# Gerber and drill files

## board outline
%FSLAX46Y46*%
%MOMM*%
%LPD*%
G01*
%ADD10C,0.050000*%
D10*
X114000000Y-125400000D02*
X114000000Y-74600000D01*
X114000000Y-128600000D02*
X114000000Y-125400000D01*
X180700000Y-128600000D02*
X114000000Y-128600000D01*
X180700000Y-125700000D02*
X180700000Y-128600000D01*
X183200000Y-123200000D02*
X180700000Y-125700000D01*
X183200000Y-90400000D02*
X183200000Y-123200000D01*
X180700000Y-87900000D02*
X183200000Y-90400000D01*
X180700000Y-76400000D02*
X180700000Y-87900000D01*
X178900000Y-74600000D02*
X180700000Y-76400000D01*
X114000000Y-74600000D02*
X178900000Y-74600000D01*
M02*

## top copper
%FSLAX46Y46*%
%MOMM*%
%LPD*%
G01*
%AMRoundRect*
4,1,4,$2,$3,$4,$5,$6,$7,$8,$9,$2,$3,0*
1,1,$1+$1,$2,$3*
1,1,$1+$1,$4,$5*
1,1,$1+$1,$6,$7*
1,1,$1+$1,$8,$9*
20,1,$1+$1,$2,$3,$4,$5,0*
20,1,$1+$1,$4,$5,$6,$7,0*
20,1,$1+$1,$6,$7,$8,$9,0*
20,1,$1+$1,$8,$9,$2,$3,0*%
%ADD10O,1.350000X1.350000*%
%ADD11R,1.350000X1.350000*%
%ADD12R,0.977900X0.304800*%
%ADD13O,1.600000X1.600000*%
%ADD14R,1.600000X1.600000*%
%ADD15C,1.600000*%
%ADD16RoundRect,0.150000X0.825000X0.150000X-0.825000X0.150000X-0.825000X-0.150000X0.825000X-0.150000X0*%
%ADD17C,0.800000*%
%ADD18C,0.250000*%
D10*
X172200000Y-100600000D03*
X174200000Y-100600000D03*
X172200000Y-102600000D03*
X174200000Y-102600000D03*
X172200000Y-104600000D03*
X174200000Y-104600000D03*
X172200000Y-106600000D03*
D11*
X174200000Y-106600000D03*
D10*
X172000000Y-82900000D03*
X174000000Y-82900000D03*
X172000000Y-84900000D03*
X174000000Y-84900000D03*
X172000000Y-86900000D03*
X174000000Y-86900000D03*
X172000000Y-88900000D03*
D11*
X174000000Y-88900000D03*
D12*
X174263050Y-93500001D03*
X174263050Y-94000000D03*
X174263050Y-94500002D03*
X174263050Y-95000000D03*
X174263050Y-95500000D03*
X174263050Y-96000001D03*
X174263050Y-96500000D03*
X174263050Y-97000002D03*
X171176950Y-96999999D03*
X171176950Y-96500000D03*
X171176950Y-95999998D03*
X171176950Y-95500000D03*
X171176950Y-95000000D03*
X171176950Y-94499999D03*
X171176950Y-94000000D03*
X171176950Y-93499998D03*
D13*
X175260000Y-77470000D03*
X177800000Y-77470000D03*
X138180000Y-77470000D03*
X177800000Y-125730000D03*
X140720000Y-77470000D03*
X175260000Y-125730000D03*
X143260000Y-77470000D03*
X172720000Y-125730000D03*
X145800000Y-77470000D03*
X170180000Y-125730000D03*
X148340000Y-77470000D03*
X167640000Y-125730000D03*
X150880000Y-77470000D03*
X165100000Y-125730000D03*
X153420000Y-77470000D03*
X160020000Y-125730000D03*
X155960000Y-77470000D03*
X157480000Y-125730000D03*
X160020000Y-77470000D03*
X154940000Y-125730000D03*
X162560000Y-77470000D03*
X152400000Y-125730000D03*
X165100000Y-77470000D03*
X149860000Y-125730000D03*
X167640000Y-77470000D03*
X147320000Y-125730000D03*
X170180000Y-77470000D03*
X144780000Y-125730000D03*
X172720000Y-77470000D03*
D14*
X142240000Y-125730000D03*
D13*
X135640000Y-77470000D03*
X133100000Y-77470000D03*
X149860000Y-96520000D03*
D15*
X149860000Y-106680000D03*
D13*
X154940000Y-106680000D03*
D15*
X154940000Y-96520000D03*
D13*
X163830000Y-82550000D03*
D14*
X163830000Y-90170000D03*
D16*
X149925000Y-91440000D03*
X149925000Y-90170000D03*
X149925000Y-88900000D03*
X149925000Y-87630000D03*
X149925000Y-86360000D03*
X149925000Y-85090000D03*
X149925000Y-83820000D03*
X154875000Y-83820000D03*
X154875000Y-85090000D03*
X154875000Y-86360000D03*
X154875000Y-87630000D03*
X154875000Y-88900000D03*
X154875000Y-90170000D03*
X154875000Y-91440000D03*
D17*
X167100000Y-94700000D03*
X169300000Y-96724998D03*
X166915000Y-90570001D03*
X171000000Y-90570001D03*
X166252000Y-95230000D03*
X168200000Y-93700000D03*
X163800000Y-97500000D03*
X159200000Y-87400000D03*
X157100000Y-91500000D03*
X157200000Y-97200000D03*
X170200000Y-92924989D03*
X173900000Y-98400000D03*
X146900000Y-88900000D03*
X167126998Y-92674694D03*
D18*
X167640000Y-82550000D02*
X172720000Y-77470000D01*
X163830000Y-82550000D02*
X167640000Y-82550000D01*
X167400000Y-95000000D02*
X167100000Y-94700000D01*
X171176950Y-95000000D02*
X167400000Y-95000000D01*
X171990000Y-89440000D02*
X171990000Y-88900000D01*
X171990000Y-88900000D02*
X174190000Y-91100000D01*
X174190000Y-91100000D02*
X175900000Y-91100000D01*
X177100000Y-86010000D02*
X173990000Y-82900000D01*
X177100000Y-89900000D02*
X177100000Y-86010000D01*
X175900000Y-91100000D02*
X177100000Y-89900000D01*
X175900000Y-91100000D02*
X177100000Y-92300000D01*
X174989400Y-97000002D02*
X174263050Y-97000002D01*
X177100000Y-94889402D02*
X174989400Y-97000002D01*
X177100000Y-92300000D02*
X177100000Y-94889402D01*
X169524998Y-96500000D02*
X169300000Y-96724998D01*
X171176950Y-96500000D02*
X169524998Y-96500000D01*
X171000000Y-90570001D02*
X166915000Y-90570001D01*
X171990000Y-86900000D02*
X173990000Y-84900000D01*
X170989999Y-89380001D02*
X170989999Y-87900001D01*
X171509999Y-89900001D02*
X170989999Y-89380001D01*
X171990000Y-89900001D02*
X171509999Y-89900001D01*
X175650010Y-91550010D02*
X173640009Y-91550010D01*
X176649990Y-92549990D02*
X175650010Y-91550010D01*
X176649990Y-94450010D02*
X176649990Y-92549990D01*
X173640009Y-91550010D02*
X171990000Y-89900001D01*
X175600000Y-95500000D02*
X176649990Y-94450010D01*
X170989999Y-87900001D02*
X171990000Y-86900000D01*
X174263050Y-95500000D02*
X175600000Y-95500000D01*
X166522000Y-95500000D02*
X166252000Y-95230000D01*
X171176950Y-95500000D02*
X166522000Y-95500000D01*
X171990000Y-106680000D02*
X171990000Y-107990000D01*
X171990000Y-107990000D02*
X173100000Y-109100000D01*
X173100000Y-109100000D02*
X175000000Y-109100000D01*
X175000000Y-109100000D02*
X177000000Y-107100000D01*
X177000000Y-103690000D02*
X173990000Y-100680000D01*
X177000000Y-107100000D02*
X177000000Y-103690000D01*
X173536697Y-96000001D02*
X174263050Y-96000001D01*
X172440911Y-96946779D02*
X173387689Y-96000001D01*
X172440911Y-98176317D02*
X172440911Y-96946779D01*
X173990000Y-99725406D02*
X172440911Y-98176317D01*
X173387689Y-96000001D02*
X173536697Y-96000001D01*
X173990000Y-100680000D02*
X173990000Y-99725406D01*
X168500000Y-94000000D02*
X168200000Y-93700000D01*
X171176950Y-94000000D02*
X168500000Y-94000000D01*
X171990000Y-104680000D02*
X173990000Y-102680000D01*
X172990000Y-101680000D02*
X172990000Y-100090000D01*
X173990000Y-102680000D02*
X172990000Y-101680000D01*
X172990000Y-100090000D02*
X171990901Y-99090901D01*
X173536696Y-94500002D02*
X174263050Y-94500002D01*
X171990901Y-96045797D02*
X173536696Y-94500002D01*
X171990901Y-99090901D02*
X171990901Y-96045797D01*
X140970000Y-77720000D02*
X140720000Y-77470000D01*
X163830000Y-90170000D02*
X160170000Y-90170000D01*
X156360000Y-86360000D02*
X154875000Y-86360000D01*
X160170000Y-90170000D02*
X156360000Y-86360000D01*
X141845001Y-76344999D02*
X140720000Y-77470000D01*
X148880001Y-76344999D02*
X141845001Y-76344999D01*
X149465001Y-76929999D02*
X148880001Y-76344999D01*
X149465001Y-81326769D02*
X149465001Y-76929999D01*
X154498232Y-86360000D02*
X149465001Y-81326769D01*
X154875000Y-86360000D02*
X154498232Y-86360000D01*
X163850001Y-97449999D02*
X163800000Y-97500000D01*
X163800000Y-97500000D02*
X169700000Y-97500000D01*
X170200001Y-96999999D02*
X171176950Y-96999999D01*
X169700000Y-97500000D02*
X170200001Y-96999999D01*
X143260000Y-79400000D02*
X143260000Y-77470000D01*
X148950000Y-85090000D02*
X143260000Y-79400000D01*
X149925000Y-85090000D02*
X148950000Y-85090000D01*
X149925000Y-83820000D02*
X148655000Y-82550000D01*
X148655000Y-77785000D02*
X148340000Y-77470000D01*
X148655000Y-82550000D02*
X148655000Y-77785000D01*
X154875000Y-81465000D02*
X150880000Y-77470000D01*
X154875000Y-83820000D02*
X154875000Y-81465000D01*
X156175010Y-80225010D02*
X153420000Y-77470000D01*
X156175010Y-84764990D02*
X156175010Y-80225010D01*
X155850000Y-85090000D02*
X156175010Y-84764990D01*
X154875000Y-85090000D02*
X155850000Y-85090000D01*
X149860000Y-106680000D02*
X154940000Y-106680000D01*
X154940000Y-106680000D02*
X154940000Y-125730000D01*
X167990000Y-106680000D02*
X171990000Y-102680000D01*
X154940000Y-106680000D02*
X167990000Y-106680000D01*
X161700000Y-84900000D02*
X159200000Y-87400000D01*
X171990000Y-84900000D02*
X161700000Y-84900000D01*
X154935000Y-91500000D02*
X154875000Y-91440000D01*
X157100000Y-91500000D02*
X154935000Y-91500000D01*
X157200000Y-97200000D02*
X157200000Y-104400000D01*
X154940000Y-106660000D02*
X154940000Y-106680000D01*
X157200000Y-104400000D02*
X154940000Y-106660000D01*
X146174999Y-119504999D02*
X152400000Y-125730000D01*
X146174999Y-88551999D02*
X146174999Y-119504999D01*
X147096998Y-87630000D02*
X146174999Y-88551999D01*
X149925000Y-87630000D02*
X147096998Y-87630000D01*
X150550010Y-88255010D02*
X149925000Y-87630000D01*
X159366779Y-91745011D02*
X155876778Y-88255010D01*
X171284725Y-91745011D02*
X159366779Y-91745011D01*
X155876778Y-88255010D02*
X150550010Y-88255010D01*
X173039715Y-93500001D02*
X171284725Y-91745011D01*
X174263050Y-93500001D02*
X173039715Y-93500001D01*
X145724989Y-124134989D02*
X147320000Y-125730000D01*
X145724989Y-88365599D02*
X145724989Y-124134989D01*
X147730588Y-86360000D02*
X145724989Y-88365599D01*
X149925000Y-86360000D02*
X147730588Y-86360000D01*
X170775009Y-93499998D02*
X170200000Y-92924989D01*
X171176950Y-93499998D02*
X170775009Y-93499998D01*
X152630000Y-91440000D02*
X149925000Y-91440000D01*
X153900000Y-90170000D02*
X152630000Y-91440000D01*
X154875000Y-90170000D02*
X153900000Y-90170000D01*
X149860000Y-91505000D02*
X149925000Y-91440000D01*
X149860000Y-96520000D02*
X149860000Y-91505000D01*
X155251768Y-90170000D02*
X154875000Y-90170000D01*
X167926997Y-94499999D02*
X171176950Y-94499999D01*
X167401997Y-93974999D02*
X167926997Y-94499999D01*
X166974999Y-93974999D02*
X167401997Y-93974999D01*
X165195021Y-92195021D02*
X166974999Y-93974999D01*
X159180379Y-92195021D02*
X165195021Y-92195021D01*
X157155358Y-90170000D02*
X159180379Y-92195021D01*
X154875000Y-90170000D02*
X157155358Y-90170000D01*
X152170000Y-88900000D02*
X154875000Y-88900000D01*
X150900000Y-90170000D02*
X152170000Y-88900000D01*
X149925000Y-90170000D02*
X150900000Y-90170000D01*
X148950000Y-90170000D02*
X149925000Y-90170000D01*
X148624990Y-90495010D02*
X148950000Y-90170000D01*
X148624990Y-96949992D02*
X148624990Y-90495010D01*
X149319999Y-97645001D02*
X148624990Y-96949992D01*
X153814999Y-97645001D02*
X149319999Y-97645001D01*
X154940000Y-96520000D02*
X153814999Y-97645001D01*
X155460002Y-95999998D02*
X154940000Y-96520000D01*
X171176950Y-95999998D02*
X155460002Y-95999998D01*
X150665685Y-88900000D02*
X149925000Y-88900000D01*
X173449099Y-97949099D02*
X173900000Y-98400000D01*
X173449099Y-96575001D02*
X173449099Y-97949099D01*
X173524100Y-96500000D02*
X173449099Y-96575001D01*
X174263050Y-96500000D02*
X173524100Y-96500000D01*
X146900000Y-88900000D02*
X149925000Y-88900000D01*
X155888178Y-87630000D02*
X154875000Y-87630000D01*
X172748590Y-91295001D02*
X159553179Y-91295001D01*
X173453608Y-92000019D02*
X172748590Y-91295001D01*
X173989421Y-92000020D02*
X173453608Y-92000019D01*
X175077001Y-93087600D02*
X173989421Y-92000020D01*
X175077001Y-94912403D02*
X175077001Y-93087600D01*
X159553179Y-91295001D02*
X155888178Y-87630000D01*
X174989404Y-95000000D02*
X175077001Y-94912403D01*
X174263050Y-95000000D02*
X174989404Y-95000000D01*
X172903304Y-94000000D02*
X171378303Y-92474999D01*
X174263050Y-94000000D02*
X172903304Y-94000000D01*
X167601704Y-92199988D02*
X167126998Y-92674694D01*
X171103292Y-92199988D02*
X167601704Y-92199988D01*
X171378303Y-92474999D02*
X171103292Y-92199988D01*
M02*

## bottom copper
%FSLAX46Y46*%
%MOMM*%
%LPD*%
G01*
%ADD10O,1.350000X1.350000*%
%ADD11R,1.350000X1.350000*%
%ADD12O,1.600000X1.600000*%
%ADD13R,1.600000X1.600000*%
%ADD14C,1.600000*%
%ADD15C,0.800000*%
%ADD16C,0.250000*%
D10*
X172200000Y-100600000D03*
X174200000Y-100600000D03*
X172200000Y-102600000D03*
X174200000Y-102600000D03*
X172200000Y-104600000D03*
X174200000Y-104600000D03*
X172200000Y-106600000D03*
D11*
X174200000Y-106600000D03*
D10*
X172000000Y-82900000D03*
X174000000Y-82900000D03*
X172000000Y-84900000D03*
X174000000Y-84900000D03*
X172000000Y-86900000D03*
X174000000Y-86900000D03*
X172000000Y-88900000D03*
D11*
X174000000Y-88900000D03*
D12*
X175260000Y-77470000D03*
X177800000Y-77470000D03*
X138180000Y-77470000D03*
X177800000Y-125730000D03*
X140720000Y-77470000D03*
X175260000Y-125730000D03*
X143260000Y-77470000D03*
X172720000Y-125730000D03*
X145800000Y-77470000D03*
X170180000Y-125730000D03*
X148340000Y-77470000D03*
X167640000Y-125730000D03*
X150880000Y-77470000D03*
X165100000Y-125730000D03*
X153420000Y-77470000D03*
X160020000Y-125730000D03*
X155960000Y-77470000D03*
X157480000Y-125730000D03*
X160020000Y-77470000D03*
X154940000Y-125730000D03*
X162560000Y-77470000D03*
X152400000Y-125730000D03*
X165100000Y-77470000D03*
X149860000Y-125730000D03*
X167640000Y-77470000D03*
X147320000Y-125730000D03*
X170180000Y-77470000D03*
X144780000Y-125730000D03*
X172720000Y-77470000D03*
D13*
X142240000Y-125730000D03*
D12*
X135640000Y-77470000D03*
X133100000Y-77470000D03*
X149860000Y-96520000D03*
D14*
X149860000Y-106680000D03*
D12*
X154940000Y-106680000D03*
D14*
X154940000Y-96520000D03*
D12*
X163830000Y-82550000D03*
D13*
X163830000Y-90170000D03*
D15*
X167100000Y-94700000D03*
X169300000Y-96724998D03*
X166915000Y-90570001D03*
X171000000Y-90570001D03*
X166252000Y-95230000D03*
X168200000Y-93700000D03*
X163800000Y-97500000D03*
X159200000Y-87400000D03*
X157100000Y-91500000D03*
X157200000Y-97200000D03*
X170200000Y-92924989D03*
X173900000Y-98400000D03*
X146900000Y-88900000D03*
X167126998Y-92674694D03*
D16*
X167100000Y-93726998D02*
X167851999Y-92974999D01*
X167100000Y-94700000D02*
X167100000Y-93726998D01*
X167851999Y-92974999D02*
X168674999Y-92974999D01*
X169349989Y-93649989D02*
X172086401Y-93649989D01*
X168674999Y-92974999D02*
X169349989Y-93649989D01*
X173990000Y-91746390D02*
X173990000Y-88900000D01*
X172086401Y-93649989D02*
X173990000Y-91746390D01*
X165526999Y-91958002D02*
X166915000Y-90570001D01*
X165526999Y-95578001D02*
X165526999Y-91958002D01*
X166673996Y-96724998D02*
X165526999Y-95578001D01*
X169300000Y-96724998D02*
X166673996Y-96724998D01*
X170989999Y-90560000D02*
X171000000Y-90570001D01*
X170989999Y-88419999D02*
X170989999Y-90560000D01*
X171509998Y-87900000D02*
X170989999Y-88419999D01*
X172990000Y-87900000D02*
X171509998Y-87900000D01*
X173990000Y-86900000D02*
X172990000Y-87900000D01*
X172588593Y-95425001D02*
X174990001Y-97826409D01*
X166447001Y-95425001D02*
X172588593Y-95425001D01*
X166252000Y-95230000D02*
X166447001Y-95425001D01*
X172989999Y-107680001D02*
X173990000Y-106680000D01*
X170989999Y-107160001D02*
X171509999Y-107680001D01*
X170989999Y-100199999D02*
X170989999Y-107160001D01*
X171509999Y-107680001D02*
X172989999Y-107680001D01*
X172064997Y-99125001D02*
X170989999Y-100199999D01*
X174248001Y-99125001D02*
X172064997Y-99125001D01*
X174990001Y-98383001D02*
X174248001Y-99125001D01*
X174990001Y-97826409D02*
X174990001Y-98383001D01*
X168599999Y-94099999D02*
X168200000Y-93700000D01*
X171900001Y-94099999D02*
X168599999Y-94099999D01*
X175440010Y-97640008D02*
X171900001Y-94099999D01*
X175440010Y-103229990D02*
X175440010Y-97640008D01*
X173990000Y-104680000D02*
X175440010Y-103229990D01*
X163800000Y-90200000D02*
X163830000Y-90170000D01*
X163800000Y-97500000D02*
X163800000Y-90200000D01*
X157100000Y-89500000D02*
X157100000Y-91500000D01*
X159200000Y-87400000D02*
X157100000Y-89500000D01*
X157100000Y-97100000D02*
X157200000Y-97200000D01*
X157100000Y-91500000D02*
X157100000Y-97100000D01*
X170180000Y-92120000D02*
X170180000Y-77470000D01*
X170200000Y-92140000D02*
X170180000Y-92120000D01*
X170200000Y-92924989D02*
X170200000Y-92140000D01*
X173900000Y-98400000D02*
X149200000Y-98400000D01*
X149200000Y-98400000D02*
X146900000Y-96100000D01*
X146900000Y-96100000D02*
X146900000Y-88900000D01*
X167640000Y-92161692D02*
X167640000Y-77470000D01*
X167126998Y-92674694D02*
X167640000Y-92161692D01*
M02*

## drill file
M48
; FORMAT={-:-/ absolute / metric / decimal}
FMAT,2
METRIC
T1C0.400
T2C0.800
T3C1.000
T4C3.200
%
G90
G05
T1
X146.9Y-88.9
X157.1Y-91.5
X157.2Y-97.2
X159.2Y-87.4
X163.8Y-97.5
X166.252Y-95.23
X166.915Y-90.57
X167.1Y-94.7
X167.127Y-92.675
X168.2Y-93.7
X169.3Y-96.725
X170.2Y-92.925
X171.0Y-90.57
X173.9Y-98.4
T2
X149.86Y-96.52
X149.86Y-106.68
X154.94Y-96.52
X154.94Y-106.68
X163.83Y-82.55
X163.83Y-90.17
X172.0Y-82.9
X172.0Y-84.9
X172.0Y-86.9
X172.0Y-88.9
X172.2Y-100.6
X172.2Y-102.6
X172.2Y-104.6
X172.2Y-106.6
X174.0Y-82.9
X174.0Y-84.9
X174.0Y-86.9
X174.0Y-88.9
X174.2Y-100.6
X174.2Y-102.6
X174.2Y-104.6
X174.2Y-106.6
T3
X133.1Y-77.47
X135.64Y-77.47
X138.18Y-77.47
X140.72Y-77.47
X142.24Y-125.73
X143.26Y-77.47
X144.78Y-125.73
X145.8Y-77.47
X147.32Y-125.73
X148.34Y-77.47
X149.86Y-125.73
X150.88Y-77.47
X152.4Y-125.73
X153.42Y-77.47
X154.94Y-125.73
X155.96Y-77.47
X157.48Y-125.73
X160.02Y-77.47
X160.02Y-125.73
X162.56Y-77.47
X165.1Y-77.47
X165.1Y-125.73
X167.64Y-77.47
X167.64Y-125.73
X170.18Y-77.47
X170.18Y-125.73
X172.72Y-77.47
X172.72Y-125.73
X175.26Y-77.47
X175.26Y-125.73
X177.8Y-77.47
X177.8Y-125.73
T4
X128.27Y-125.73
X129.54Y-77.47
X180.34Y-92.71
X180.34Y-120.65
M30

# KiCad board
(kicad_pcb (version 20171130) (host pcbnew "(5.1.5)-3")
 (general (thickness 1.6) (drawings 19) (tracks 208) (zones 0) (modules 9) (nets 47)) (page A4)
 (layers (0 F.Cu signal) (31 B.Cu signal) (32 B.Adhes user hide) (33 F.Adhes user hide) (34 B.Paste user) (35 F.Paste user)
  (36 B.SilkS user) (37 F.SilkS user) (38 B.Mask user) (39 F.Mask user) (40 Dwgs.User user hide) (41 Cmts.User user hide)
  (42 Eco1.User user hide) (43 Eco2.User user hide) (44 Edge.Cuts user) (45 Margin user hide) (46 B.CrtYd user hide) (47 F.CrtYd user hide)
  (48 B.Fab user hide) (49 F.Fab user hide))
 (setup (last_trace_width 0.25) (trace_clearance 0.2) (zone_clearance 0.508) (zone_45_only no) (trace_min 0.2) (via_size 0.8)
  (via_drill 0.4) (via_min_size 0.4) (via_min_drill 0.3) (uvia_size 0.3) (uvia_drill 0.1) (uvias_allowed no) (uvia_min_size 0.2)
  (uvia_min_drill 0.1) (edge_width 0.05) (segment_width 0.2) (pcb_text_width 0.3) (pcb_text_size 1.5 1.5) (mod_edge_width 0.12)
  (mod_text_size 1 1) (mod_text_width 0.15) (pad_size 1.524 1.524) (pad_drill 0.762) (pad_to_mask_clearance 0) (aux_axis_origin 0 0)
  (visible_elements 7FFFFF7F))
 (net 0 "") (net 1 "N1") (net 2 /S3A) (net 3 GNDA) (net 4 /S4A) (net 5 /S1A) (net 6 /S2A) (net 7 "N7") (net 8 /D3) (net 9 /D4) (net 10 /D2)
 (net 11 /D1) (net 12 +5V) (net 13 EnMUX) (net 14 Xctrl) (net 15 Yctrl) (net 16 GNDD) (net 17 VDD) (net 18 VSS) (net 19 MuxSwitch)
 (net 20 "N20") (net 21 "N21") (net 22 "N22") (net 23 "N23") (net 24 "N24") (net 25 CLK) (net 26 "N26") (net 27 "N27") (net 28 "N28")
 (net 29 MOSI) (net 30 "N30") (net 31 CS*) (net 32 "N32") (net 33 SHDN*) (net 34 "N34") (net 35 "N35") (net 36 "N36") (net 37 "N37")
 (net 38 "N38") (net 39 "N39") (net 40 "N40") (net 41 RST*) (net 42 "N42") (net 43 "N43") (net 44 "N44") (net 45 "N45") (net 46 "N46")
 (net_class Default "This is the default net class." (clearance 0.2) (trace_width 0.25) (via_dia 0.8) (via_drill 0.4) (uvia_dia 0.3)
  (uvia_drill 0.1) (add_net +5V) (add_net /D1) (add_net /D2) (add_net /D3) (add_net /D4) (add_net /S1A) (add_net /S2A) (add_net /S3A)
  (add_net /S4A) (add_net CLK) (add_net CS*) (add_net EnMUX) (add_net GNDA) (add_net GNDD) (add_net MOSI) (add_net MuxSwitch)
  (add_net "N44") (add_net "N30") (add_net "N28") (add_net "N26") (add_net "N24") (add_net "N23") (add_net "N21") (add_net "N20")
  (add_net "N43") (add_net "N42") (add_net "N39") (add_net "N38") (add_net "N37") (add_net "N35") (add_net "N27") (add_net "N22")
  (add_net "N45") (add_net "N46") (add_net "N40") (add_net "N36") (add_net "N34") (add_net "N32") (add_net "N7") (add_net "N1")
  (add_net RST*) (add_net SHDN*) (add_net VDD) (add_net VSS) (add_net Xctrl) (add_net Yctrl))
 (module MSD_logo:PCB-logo (layer F.Cu) (at 128.7 102 90)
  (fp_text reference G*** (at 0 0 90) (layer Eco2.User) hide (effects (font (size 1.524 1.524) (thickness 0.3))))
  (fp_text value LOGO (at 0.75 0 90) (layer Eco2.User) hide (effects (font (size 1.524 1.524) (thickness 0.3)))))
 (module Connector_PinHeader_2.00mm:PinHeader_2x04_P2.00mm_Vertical (layer F.Cu) (at 174.2 106.6 180)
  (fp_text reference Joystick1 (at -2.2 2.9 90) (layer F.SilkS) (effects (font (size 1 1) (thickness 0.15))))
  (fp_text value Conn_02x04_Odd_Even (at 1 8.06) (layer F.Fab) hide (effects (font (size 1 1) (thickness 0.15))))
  (pad 8 thru_hole oval (at 2 6 180) (size 1.35 1.35) (drill 0.8) (layers *.Cu *.Mask) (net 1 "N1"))
  (pad 7 thru_hole oval (at 0 6 180) (size 1.35 1.35) (drill 0.8) (layers *.Cu *.Mask) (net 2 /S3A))
  (pad 6 thru_hole oval (at 2 4 180) (size 1.35 1.35) (drill 0.8) (layers *.Cu *.Mask) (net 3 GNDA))
  (pad 5 thru_hole oval (at 0 4 180) (size 1.35 1.35) (drill 0.8) (layers *.Cu *.Mask) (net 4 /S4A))
  (pad 4 thru_hole oval (at 2 2 180) (size 1.35 1.35) (drill 0.8) (layers *.Cu *.Mask) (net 4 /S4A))
  (pad 3 thru_hole oval (at 0 2 180) (size 1.35 1.35) (drill 0.8) (layers *.Cu *.Mask) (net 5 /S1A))
  (pad 2 thru_hole oval (at 2 0 180) (size 1.35 1.35) (drill 0.8) (layers *.Cu *.Mask) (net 2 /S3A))
  (pad 1 thru_hole rect (at 0 0 180) (size 1.35 1.35) (drill 0.8) (layers *.Cu *.Mask) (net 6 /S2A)))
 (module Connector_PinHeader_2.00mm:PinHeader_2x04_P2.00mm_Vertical (layer F.Cu) (at 174 88.9 180)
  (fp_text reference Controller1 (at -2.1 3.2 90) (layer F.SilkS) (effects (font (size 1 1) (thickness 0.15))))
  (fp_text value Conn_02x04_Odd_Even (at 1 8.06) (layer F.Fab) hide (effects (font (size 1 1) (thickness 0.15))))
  (pad 8 thru_hole oval (at 2 6 180) (size 1.35 1.35) (drill 0.8) (layers *.Cu *.Mask) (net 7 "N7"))
  (pad 7 thru_hole oval (at 0 6 180) (size 1.35 1.35) (drill 0.8) (layers *.Cu *.Mask) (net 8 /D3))
  (pad 6 thru_hole oval (at 2 4 180) (size 1.35 1.35) (drill 0.8) (layers *.Cu *.Mask) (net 3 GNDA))
  (pad 5 thru_hole oval (at 0 4 180) (size 1.35 1.35) (drill 0.8) (layers *.Cu *.Mask) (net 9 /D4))
  (pad 4 thru_hole oval (at 2 2 180) (size 1.35 1.35) (drill 0.8) (layers *.Cu *.Mask) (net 9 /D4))
  (pad 3 thru_hole oval (at 0 2 180) (size 1.35 1.35) (drill 0.8) (layers *.Cu *.Mask) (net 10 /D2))
  (pad 2 thru_hole oval (at 2 0 180) (size 1.35 1.35) (drill 0.8) (layers *.Cu *.Mask) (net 8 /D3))
  (pad 1 thru_hole rect (at 0 0 180) (size 1.35 1.35) (drill 0.8) (layers *.Cu *.Mask) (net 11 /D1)))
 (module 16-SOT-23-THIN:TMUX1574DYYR (layer F.Cu) (at 172.72 95.25)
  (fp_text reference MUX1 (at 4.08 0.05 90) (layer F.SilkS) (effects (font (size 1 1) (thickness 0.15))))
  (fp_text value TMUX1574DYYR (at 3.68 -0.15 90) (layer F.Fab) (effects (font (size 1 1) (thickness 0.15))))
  (pad 16 smd rect (at 1.54305 -1.749999) (size 0.9779 0.3048) (layers F.Cu F.Paste F.Mask) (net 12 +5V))
  (pad 15 smd rect (at 1.54305 -1.25) (size 0.9779 0.3048) (layers F.Cu F.Paste F.Mask) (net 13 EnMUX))
  (pad 14 smd rect (at 1.54305 -0.749998) (size 0.9779 0.3048) (layers F.Cu F.Paste F.Mask) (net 4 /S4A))
  (pad 13 smd rect (at 1.54305 -0.25) (size 0.9779 0.3048) (layers F.Cu F.Paste F.Mask) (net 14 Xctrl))
  (pad 12 smd rect (at 1.54305 0.25) (size 0.9779 0.3048) (layers F.Cu F.Paste F.Mask) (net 9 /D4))
  (pad 11 smd rect (at 1.54305 0.750001) (size 0.9779 0.3048) (layers F.Cu F.Paste F.Mask) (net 2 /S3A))
  (pad 10 smd rect (at 1.54305 1.25) (size 0.9779 0.3048) (layers F.Cu F.Paste F.Mask) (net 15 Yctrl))
  (pad 9 smd rect (at 1.54305 1.750002) (size 0.9779 0.3048) (layers F.Cu F.Paste F.Mask) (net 8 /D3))
  (pad 8 smd rect (at -1.54305 1.749999) (size 0.9779 0.3048) (layers F.Cu F.Paste F.Mask) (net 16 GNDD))
  (pad 7 smd rect (at -1.54305 1.25) (size 0.9779 0.3048) (layers F.Cu F.Paste F.Mask) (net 10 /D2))
  (pad 6 smd rect (at -1.54305 0.749998) (size 0.9779 0.3048) (layers F.Cu F.Paste F.Mask) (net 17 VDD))
  (pad 5 smd rect (at -1.54305 0.25) (size 0.9779 0.3048) (layers F.Cu F.Paste F.Mask) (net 6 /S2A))
  (pad 4 smd rect (at -1.54305 -0.25) (size 0.9779 0.3048) (layers F.Cu F.Paste F.Mask) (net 11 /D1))
  (pad 3 smd rect (at -1.54305 -0.750001) (size 0.9779 0.3048) (layers F.Cu F.Paste F.Mask) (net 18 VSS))
  (pad 2 smd rect (at -1.54305 -1.25) (size 0.9779 0.3048) (layers F.Cu F.Paste F.Mask) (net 5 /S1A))
  (pad 1 smd rect (at -1.54305 -1.750002) (size 0.9779 0.3048) (layers F.Cu F.Paste F.Mask) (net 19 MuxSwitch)))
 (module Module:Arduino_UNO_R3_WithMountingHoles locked (layer B.Cu) (at 142.24 125.73)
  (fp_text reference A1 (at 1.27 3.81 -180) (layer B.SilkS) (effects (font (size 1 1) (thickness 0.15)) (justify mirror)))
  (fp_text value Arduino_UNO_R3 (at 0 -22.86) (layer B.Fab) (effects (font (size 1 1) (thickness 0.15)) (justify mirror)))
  (pad "" np_thru_hole circle (at 38.1 -5.08 270) (size 3.2 3.2) (drill 3.2) (layers *.Cu *.Mask))
  (pad "" np_thru_hole circle (at 38.1 -33.02 270) (size 3.2 3.2) (drill 3.2) (layers *.Cu *.Mask))
  (pad "" np_thru_hole circle (at -12.7 -48.26 270) (size 3.2 3.2) (drill 3.2) (layers *.Cu *.Mask))
  (pad "" np_thru_hole circle (at -13.97 0 270) (size 3.2 3.2) (drill 3.2) (layers *.Cu *.Mask))
  (pad 16 thru_hole oval (at 33.02 -48.26 270) (size 1.6 1.6) (drill 1) (layers *.Cu *.Mask) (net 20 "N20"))
  (pad 15 thru_hole oval (at 35.56 -48.26 270) (size 1.6 1.6) (drill 1) (layers *.Cu *.Mask) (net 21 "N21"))
  (pad 30 thru_hole oval (at -4.06 -48.26 270) (size 1.6 1.6) (drill 1) (layers *.Cu *.Mask) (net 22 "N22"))
  (pad 14 thru_hole oval (at 35.56 0 270) (size 1.6 1.6) (drill 1) (layers *.Cu *.Mask) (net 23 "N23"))
  (pad 29 thru_hole oval (at -1.52 -48.26 270) (size 1.6 1.6) (drill 1) (layers *.Cu *.Mask) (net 16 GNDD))
  (pad 13 thru_hole oval (at 33.02 0 270) (size 1.6 1.6) (drill 1) (layers *.Cu *.Mask) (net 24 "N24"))
  (pad 28 thru_hole oval (at 1.02 -48.26 270) (size 1.6 1.6) (drill 1) (layers *.Cu *.Mask) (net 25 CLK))
  (pad 12 thru_hole oval (at 30.48 0 270) (size 1.6 1.6) (drill 1) (layers *.Cu *.Mask) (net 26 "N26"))
  (pad 27 thru_hole oval (at 3.56 -48.26 270) (size 1.6 1.6) (drill 1) (layers *.Cu *.Mask) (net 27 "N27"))
  (pad 11 thru_hole oval (at 27.94 0 270) (size 1.6 1.6) (drill 1) (layers *.Cu *.Mask) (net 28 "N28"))
  (pad 26 thru_hole oval (at 6.1 -48.26 270) (size 1.6 1.6) (drill 1) (layers *.Cu *.Mask) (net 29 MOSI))
  (pad 10 thru_hole oval (at 25.4 0 270) (size 1.6 1.6) (drill 1) (layers *.Cu *.Mask) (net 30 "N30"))
  (pad 25 thru_hole oval (at 8.64 -48.26 270) (size 1.6 1.6) (drill 1) (layers *.Cu *.Mask) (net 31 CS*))
  (pad 9 thru_hole oval (at 22.86 0 270) (size 1.6 1.6) (drill 1) (layers *.Cu *.Mask) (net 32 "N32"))
  (pad 24 thru_hole oval (at 11.18 -48.26 270) (size 1.6 1.6) (drill 1) (layers *.Cu *.Mask) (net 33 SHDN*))
  (pad 8 thru_hole oval (at 17.78 0 270) (size 1.6 1.6) (drill 1) (layers *.Cu *.Mask) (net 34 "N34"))
  (pad 23 thru_hole oval (at 13.72 -48.26 270) (size 1.6 1.6) (drill 1) (layers *.Cu *.Mask) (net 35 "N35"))
  (pad 7 thru_hole oval (at 15.24 0 270) (size 1.6 1.6) (drill 1) (layers *.Cu *.Mask) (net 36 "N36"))
  (pad 22 thru_hole oval (at 17.78 -48.26 270) (size 1.6 1.6) (drill 1) (layers *.Cu *.Mask) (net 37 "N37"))
  (pad 6 thru_hole oval (at 12.7 0 270) (size 1.6 1.6) (drill 1) (layers *.Cu *.Mask) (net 3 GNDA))
  (pad 21 thru_hole oval (at 20.32 -48.26 270) (size 1.6 1.6) (drill 1) (layers *.Cu *.Mask) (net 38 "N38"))
  (pad 5 thru_hole oval (at 10.16 0 270) (size 1.6 1.6) (drill 1) (layers *.Cu *.Mask) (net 12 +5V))
  (pad 20 thru_hole oval (at 22.86 -48.26 270) (size 1.6 1.6) (drill 1) (layers *.Cu *.Mask) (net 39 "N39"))
  (pad 4 thru_hole oval (at 7.62 0 270) (size 1.6 1.6) (drill 1) (layers *.Cu *.Mask) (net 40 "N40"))
  (pad 19 thru_hole oval (at 25.4 -48.26 270) (size 1.6 1.6) (drill 1) (layers *.Cu *.Mask) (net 13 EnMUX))
  (pad 3 thru_hole oval (at 5.08 0 270) (size 1.6 1.6) (drill 1) (layers *.Cu *.Mask) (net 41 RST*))
  (pad 18 thru_hole oval (at 27.94 -48.26 270) (size 1.6 1.6) (drill 1) (layers *.Cu *.Mask) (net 19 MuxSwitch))
  (pad 2 thru_hole oval (at 2.54 0 270) (size 1.6 1.6) (drill 1) (layers *.Cu *.Mask) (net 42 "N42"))
  (pad 17 thru_hole oval (at 30.48 -48.26 270) (size 1.6 1.6) (drill 1) (layers *.Cu *.Mask) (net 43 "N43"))
  (pad 1 thru_hole rect (at 0 0 270) (size 1.6 1.6) (drill 1) (layers *.Cu *.Mask) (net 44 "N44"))
  (pad 31 thru_hole oval (at -6.6 -48.26 270) (size 1.6 1.6) (drill 1) (layers *.Cu *.Mask) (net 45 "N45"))
  (pad 32 thru_hole oval (at -9.14 -48.26 270) (size 1.6 1.6) (drill 1) (layers *.Cu *.Mask) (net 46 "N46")))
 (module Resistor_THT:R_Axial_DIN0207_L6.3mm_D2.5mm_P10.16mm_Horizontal (layer F.Cu) (at 149.86 106.68 90)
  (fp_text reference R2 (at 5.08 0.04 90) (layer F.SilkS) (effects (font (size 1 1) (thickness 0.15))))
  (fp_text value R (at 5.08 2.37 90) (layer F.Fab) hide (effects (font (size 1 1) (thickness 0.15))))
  (pad 2 thru_hole oval (at 10.16 0 90) (size 1.6 1.6) (drill 0.8) (layers *.Cu *.Mask) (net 18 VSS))
  (pad 1 thru_hole circle (at 0 0 90) (size 1.6 1.6) (drill 0.8) (layers *.Cu *.Mask) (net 3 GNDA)))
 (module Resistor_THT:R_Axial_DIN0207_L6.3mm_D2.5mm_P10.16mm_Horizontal (layer F.Cu) (at 154.94 96.52 270)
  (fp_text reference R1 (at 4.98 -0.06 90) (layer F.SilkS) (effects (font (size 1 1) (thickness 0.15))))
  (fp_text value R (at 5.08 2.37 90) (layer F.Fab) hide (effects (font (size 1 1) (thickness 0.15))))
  (pad 2 thru_hole oval (at 10.16 0 270) (size 1.6 1.6) (drill 0.8) (layers *.Cu *.Mask) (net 3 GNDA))
  (pad 1 thru_hole circle (at 0 0 270) (size 1.6 1.6) (drill 0.8) (layers *.Cu *.Mask) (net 17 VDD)))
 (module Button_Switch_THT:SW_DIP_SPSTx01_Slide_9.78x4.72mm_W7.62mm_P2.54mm (layer F.Cu) (at 163.83 90.17 90)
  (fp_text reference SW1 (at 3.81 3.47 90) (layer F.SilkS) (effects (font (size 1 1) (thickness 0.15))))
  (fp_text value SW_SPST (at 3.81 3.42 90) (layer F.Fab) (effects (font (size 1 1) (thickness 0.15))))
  (pad 2 thru_hole oval (at 7.62 0 90) (size 1.6 1.6) (drill 0.8) (layers *.Cu *.Mask) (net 43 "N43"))
  (pad 1 thru_hole rect (at 0 0 90) (size 1.6 1.6) (drill 0.8) (layers *.Cu *.Mask) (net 16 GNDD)))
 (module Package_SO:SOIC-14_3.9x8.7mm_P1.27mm (layer F.Cu) (at 152.4 87.63 180)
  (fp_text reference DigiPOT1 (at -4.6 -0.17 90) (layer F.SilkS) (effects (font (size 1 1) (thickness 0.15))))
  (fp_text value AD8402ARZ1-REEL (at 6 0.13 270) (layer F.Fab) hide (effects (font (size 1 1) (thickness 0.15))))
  (pad 14 smd roundrect (at 2.475 -3.81 180) (size 1.95 0.6) (layers F.Cu F.Paste F.Mask) (roundrect_rratio 0.25) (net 18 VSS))
  (pad 13 smd roundrect (at 2.475 -2.54 180) (size 1.95 0.6) (layers F.Cu F.Paste F.Mask) (roundrect_rratio 0.25) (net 17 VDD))
  (pad 12 smd roundrect (at 2.475 -1.27 180) (size 1.95 0.6) (layers F.Cu F.Paste F.Mask) (roundrect_rratio 0.25) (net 15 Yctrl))
  (pad 11 smd roundrect (at 2.475 0 180) (size 1.95 0.6) (layers F.Cu F.Paste F.Mask) (roundrect_rratio 0.25) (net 12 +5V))
  (pad 10 smd roundrect (at 2.475 1.27 180) (size 1.95 0.6) (layers F.Cu F.Paste F.Mask) (roundrect_rratio 0.25) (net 41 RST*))
  (pad 9 smd roundrect (at 2.475 2.54 180) (size 1.95 0.6) (layers F.Cu F.Paste F.Mask) (roundrect_rratio 0.25) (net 25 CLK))
  (pad 8 smd roundrect (at 2.475 3.81 180) (size 1.95 0.6) (layers F.Cu F.Paste F.Mask) (roundrect_rratio 0.25) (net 29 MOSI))
  (pad 7 smd roundrect (at -2.475 3.81 180) (size 1.95 0.6) (layers F.Cu F.Paste F.Mask) (roundrect_rratio 0.25) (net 31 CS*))
  (pad 6 smd roundrect (at -2.475 2.54 180) (size 1.95 0.6) (layers F.Cu F.Paste F.Mask) (roundrect_rratio 0.25) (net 33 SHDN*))
  (pad 5 smd roundrect (at -2.475 1.27 180) (size 1.95 0.6) (layers F.Cu F.Paste F.Mask) (roundrect_rratio 0.25) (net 16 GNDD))
  (pad 4 smd roundrect (at -2.475 0 180) (size 1.95 0.6) (layers F.Cu F.Paste F.Mask) (roundrect_rratio 0.25) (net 14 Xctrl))
  (pad 3 smd roundrect (at -2.475 -1.27 180) (size 1.95 0.6) (layers F.Cu F.Paste F.Mask) (roundrect_rratio 0.25) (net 17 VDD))
  (pad 2 smd roundrect (at -2.475 -2.54 180) (size 1.95 0.6) (layers F.Cu F.Paste F.Mask) (roundrect_rratio 0.25) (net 18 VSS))
  (pad 1 smd roundrect (at -2.475 -3.81 180) (size 1.95 0.6) (layers F.Cu F.Paste F.Mask) (roundrect_rratio 0.25) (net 3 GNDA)))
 (gr_line (start 114 125.4) (end 114 74.6) (layer Edge.Cuts) (width 0.05))
 (gr_line (start 114 128.6) (end 114 125.4) (layer Edge.Cuts) (width 0.05))
 (gr_line (start 180.7 128.6) (end 114 128.6) (layer Edge.Cuts) (width 0.05))
 (gr_line (start 180.7 125.7) (end 180.7 128.6) (layer Edge.Cuts) (width 0.05))
 (gr_line (start 183.2 123.2) (end 180.7 125.7) (layer Edge.Cuts) (width 0.05))
 (gr_line (start 183.2 90.4) (end 183.2 123.2) (layer Edge.Cuts) (width 0.05))
 (gr_line (start 180.7 87.9) (end 183.2 90.4) (layer Edge.Cuts) (width 0.05))
 (gr_line (start 180.7 76.4) (end 180.7 87.9) (layer Edge.Cuts) (width 0.05))
 (gr_line (start 178.9 74.6) (end 180.7 76.4) (layer Edge.Cuts) (width 0.05))
 (gr_line (start 114 74.6) (end 178.9 74.6) (layer Edge.Cuts) (width 0.05))
 (segment (start 167.64 82.55) (end 172.72 77.47) (width 0.25) (layer F.Cu) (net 43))
 (segment (start 163.83 82.55) (end 167.64 82.55) (width 0.25) (layer F.Cu) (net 43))
 (via (at 167.1 94.7) (size 0.8) (drill 0.4) (layers F.Cu B.Cu) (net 11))
 (segment (start 167.4 95) (end 167.1 94.7) (width 0.25) (layer F.Cu) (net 11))
 (segment (start 171.17695 95) (end 167.4 95) (width 0.25) (layer F.Cu) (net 11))
 (segment (start 167.1 93.726998) (end 167.851999 92.974999) (width 0.25) (layer B.Cu) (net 11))
 (segment (start 167.1 94.7) (end 167.1 93.726998) (width 0.25) (layer B.Cu) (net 11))
 (segment (start 167.851999 92.974999) (end 168.674999 92.974999) (width 0.25) (layer B.Cu) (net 11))
 (segment (start 169.349989 93.649989) (end 172.086401 93.649989) (width 0.25) (layer B.Cu) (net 11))
 (segment (start 168.674999 92.974999) (end 169.349989 93.649989) (width 0.25) (layer B.Cu) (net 11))
 (segment (start 173.99 91.74639) (end 173.99 88.9) (width 0.25) (layer B.Cu) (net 11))
 (segment (start 172.086401 93.649989) (end 173.99 91.74639) (width 0.25) (layer B.Cu) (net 11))
 (segment (start 171.99 89.44) (end 171.99 88.9) (width 0.25) (layer F.Cu) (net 8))
 (segment (start 171.99 88.9) (end 174.19 91.1) (width 0.25) (layer F.Cu) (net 8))
 (segment (start 174.19 91.1) (end 175.9 91.1) (width 0.25) (layer F.Cu) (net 8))
 (segment (start 177.1 86.01) (end 173.99 82.9) (width 0.25) (layer F.Cu) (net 8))
 (segment (start 177.1 89.9) (end 177.1 86.01) (width 0.25) (layer F.Cu) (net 8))
 (segment (start 175.9 91.1) (end 177.1 89.9) (width 0.25) (layer F.Cu) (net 8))
 (segment (start 175.9 91.1) (end 177.1 92.3) (width 0.25) (layer F.Cu) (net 8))
 (segment (start 174.9894 97.000002) (end 174.26305 97.000002) (width 0.25) (layer F.Cu) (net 8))
 (segment (start 177.1 94.889402) (end 174.9894 97.000002) (width 0.25) (layer F.Cu) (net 8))
 (segment (start 177.1 92.3) (end 177.1 94.889402) (width 0.25) (layer F.Cu) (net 8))
 (via (at 169.3 96.724998) (size 0.8) (drill 0.4) (layers F.Cu B.Cu) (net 10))
 (segment (start 169.524998 96.5) (end 169.3 96.724998) (width 0.25) (layer F.Cu) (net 10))
 (segment (start 171.17695 96.5) (end 169.524998 96.5) (width 0.25) (layer F.Cu) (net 10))
 (segment (start 165.526999 91.958002) (end 166.915 90.570001) (width 0.25) (layer B.Cu) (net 10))
 (via (at 166.915 90.570001) (size 0.8) (drill 0.4) (layers F.Cu B.Cu) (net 10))
 (segment (start 165.526999 95.578001) (end 165.526999 91.958002) (width 0.25) (layer B.Cu) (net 10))
 (segment (start 166.673996 96.724998) (end 165.526999 95.578001) (width 0.25) (layer B.Cu) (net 10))
 (segment (start 169.3 96.724998) (end 166.673996 96.724998) (width 0.25) (layer B.Cu) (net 10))
 (via (at 171 90.570001) (size 0.8) (drill 0.4) (layers F.Cu B.Cu) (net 10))
 (segment (start 170.989999 90.56) (end 171 90.570001) (width 0.25) (layer B.Cu) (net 10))
 (segment (start 170.989999 88.419999) (end 170.989999 90.56) (width 0.25) (layer B.Cu) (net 10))
 (segment (start 171.509998 87.9) (end 170.989999 88.419999) (width 0.25) (layer B.Cu) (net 10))
 (segment (start 172.99 87.9) (end 171.509998 87.9) (width 0.25) (layer B.Cu) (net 10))
 (segment (start 173.99 86.9) (end 172.99 87.9) (width 0.25) (layer B.Cu) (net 10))
 (segment (start 171 90.570001) (end 166.915 90.570001) (width 0.25) (layer F.Cu) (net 10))
 (segment (start 171.99 86.9) (end 173.99 84.9) (width 0.25) (layer F.Cu) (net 9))
 (segment (start 170.989999 89.380001) (end 170.989999 87.900001) (width 0.25) (layer F.Cu) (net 9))
 (segment (start 171.509999 89.900001) (end 170.989999 89.380001) (width 0.25) (layer F.Cu) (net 9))
 (segment (start 171.99 89.900001) (end 171.509999 89.900001) (width 0.25) (layer F.Cu) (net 9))
 (segment (start 175.65001 91.55001) (end 173.640009 91.55001) (width 0.25) (layer F.Cu) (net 9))
 (segment (start 176.64999 92.54999) (end 175.65001 91.55001) (width 0.25) (layer F.Cu) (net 9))
 (segment (start 176.64999 94.45001) (end 176.64999 92.54999) (width 0.25) (layer F.Cu) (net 9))
 (segment (start 173.640009 91.55001) (end 171.99 89.900001) (width 0.25) (layer F.Cu) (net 9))
 (segment (start 175.6 95.5) (end 176.64999 94.45001) (width 0.25) (layer F.Cu) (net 9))
 (segment (start 170.989999 87.900001) (end 171.99 86.9) (width 0.25) (layer F.Cu) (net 9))
 (segment (start 174.26305 95.5) (end 175.6 95.5) (width 0.25) (layer F.Cu) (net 9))
 (via (at 166.252 95.23) (size 0.8) (drill 0.4) (layers F.Cu B.Cu) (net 6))
 (segment (start 166.522 95.5) (end 166.252 95.23) (width 0.25) (layer F.Cu) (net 6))
 (segment (start 171.17695 95.5) (end 166.522 95.5) (width 0.25) (layer F.Cu) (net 6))
 (segment (start 172.588593 95.425001) (end 174.990001 97.826409) (width 0.25) (layer B.Cu) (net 6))
 (segment (start 166.447001 95.425001) (end 172.588593 95.425001) (width 0.25) (layer B.Cu) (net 6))
 (segment (start 166.252 95.23) (end 166.447001 95.425001) (width 0.25) (layer B.Cu) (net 6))
 (segment (start 172.989999 107.680001) (end 173.99 106.68) (width 0.25) (layer B.Cu) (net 6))
 (segment (start 170.989999 107.160001) (end 171.509999 107.680001) (width 0.25) (layer B.Cu) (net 6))
 (segment (start 170.989999 100.199999) (end 170.989999 107.160001) (width 0.25) (layer B.Cu) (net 6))
 (segment (start 171.509999 107.680001) (end 172.989999 107.680001) (width 0.25) (layer B.Cu) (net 6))
 (segment (start 172.064997 99.125001) (end 170.989999 100.199999) (width 0.25) (layer B.Cu) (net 6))
 (segment (start 174.248001 99.125001) (end 172.064997 99.125001) (width 0.25) (layer B.Cu) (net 6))
 (segment (start 174.990001 98.383001) (end 174.248001 99.125001) (width 0.25) (layer B.Cu) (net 6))
 (segment (start 174.990001 97.826409) (end 174.990001 98.383001) (width 0.25) (layer B.Cu) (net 6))
 (segment (start 171.99 106.68) (end 171.99 107.99) (width 0.25) (layer F.Cu) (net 2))
 (segment (start 171.99 107.99) (end 173.1 109.1) (width 0.25) (layer F.Cu) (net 2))
 (segment (start 173.1 109.1) (end 175 109.1) (width 0.25) (layer F.Cu) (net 2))
 (segment (start 175 109.1) (end 177 107.1) (width 0.25) (layer F.Cu) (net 2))
 (segment (start 177 103.69) (end 173.99 100.68) (width 0.25) (layer F.Cu) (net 2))
 (segment (start 177 107.1) (end 177 103.69) (width 0.25) (layer F.Cu) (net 2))
 (segment (start 173.536697 96.000001) (end 174.26305 96.000001) (width 0.25) (layer F.Cu) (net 2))
 (segment (start 172.440911 96.946779) (end 173.387689 96.000001) (width 0.25) (layer F.Cu) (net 2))
 (segment (start 172.440911 98.176317) (end 172.440911 96.946779) (width 0.25) (layer F.Cu) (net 2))
 (segment (start 173.99 99.725406) (end 172.440911 98.176317) (width 0.25) (layer F.Cu) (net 2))
 (segment (start 173.387689 96.000001) (end 173.536697 96.000001) (width 0.25) (layer F.Cu) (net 2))
 (segment (start 173.99 100.68) (end 173.99 99.725406) (width 0.25) (layer F.Cu) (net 2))
 (via (at 168.2 93.7) (size 0.8) (drill 0.4) (layers F.Cu B.Cu) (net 5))
 (segment (start 168.5 94) (end 168.2 93.7) (width 0.25) (layer F.Cu) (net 5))
 (segment (start 171.17695 94) (end 168.5 94) (width 0.25) (layer F.Cu) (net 5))
 (segment (start 168.599999 94.099999) (end 168.2 93.7) (width 0.25) (layer B.Cu) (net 5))
 (segment (start 171.900001 94.099999) (end 168.599999 94.099999) (width 0.25) (layer B.Cu) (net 5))
 (segment (start 175.44001 97.640008) (end 171.900001 94.099999) (width 0.25) (layer B.Cu) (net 5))
 (segment (start 175.44001 103.22999) (end 175.44001 97.640008) (width 0.25) (layer B.Cu) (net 5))
 (segment (start 173.99 104.68) (end 175.44001 103.22999) (width 0.25) (layer B.Cu) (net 5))
 (segment (start 171.99 104.68) (end 173.99 102.68) (width 0.25) (layer F.Cu) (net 4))
 (segment (start 172.99 101.68) (end 172.99 100.09) (width 0.25) (layer F.Cu) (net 4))
 (segment (start 173.99 102.68) (end 172.99 101.68) (width 0.25) (layer F.Cu) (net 4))
 (segment (start 172.99 100.09) (end 171.990901 99.090901) (width 0.25) (layer F.Cu) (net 4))
 (segment (start 173.536696 94.500002) (end 174.26305 94.500002) (width 0.25) (layer F.Cu) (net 4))
 (segment (start 171.990901 96.045797) (end 173.536696 94.500002) (width 0.25) (layer F.Cu) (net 4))
 (segment (start 171.990901 99.090901) (end 171.990901 96.045797) (width 0.25) (layer F.Cu) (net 4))
 (segment (start 140.97 77.72) (end 140.72 77.47) (width 0.25) (layer F.Cu) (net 16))
 (segment (start 163.83 90.17) (end 160.17 90.17) (width 0.25) (layer F.Cu) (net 16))
 (segment (start 156.36 86.36) (end 154.875 86.36) (width 0.25) (layer F.Cu) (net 16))
 (segment (start 160.17 90.17) (end 156.36 86.36) (width 0.25) (layer F.Cu) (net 16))
 (segment (start 141.845001 76.344999) (end 140.72 77.47) (width 0.25) (layer F.Cu) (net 16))
 (segment (start 148.880001 76.344999) (end 141.845001 76.344999) (width 0.25) (layer F.Cu) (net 16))
 (segment (start 149.465001 76.929999) (end 148.880001 76.344999) (width 0.25) (layer F.Cu) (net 16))
 (segment (start 149.465001 81.326769) (end 149.465001 76.929999) (width 0.25) (layer F.Cu) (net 16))
 (segment (start 154.498232 86.36) (end 149.465001 81.326769) (width 0.25) (layer F.Cu) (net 16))
 (segment (start 154.875 86.36) (end 154.498232 86.36) (width 0.25) (layer F.Cu) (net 16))
 (via (at 163.8 97.5) (size 0.8) (drill 0.4) (layers F.Cu B.Cu) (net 16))
 (segment (start 163.850001 97.449999) (end 163.8 97.5) (width 0.25) (layer F.Cu) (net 16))
 (segment (start 163.8 90.2) (end 163.83 90.17) (width 0.25) (layer B.Cu) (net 16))
 (segment (start 163.8 97.5) (end 163.8 90.2) (width 0.25) (layer B.Cu) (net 16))
 (segment (start 163.8 97.5) (end 169.7 97.5) (width 0.25) (layer F.Cu) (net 16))
 (segment (start 170.200001 96.999999) (end 171.17695 96.999999) (width 0.25) (layer F.Cu) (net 16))
 (segment (start 169.7 97.5) (end 170.200001 96.999999) (width 0.25) (layer F.Cu) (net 16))
 (segment (start 143.26 79.4) (end 143.26 77.47) (width 0.25) (layer F.Cu) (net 25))
 (segment (start 148.95 85.09) (end 143.26 79.4) (width 0.25) (layer F.Cu) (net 25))
 (segment (start 149.925 85.09) (end 148.95 85.09) (width 0.25) (layer F.Cu) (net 25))
 (segment (start 149.925 83.82) (end 148.655 82.55) (width 0.25) (layer F.Cu) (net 29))
 (segment (start 148.655 77.785) (end 148.34 77.47) (width 0.25) (layer F.Cu) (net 29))
 (segment (start 148.655 82.55) (end 148.655 77.785) (width 0.25) (layer F.Cu) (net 29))
 (segment (start 154.875 81.465) (end 150.88 77.47) (width 0.25) (layer F.Cu) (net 31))
 (segment (start 154.875 83.82) (end 154.875 81.465) (width 0.25) (layer F.Cu) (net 31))
 (segment (start 156.17501 80.22501) (end 153.42 77.47) (width 0.25) (layer F.Cu) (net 33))
 (segment (start 156.17501 84.76499) (end 156.17501 80.22501) (width 0.25) (layer F.Cu) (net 33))
 (segment (start 155.85 85.09) (end 156.17501 84.76499) (width 0.25) (layer F.Cu) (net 33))
 (segment (start 154.875 85.09) (end 155.85 85.09) (width 0.25) (layer F.Cu) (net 33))
 (segment (start 149.86 106.68) (end 154.94 106.68) (width 0.25) (layer F.Cu) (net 3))
 (segment (start 154.94 106.68) (end 154.94 125.73) (width 0.25) (layer F.Cu) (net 3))
 (segment (start 167.99 106.68) (end 171.99 102.68) (width 0.25) (layer F.Cu) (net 3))
 (segment (start 154.94 106.68) (end 167.99 106.68) (width 0.25) (layer F.Cu) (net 3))
 (via (at 159.2 87.4) (size 0.8) (drill 0.4) (layers F.Cu B.Cu) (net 3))
 (segment (start 161.7 84.9) (end 159.2 87.4) (width 0.25) (layer F.Cu) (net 3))
 (segment (start 171.99 84.9) (end 161.7 84.9) (width 0.25) (layer F.Cu) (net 3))
 (via (at 157.1 91.5) (size 0.8) (drill 0.4) (layers F.Cu B.Cu) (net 3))
 (segment (start 157.1 89.5) (end 157.1 91.5) (width 0.25) (layer B.Cu) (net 3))
 (segment (start 159.2 87.4) (end 157.1 89.5) (width 0.25) (layer B.Cu) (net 3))
 (segment (start 154.935 91.5) (end 154.875 91.44) (width 0.25) (layer F.Cu) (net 3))
 (segment (start 157.1 91.5) (end 154.935 91.5) (width 0.25) (layer F.Cu) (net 3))
 (via (at 157.2 97.2) (size 0.8) (drill 0.4) (layers F.Cu B.Cu) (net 3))
 (segment (start 157.1 97.1) (end 157.2 97.2) (width 0.25) (layer B.Cu) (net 3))
 (segment (start 157.1 91.5) (end 157.1 97.1) (width 0.25) (layer B.Cu) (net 3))
 (segment (start 157.2 97.2) (end 157.2 104.4) (width 0.25) (layer F.Cu) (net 3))
 (segment (start 154.94 106.66) (end 154.94 106.68) (width 0.25) (layer F.Cu) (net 3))
 (segment (start 157.2 104.4) (end 154.94 106.66) (width 0.25) (layer F.Cu) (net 3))
 (segment (start 146.174999 119.504999) (end 152.4 125.73) (width 0.25) (layer F.Cu) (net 12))
 (segment (start 146.174999 88.551999) (end 146.174999 119.504999) (width 0.25) (layer F.Cu) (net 12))
 (segment (start 147.096998 87.63) (end 146.174999 88.551999) (width 0.25) (layer F.Cu) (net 12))
 (segment (start 149.925 87.63) (end 147.096998 87.63) (width 0.25) (layer F.Cu) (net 12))
 (segment (start 150.55001 88.25501) (end 149.925 87.63) (width 0.25) (layer F.Cu) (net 12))
 (segment (start 159.366779 91.745011) (end 155.876778 88.25501) (width 0.25) (layer F.Cu) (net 12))
 (segment (start 171.284725 91.745011) (end 159.366779 91.745011) (width 0.25) (layer F.Cu) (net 12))
 (segment (start 155.876778 88.25501) (end 150.55001 88.25501) (width 0.25) (layer F.Cu) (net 12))
 (segment (start 173.039715 93.500001) (end 171.284725 91.745011) (width 0.25) (layer F.Cu) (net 12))
 (segment (start 174.26305 93.500001) (end 173.039715 93.500001) (width 0.25) (layer F.Cu) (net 12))
 (segment (start 145.724989 124.134989) (end 147.32 125.73) (width 0.25) (layer F.Cu) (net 41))
 (segment (start 145.724989 88.365599) (end 145.724989 124.134989) (width 0.25) (layer F.Cu) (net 41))
 (segment (start 147.730588 86.36) (end 145.724989 88.365599) (width 0.25) (layer F.Cu) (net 41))
 (segment (start 149.925 86.36) (end 147.730588 86.36) (width 0.25) (layer F.Cu) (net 41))
 (segment (start 170.18 92.12) (end 170.18 77.47) (width 0.25) (layer B.Cu) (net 19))
 (via (at 170.2 92.924989) (size 0.8) (drill 0.4) (layers F.Cu B.Cu) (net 19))
 (segment (start 170.775009 93.499998) (end 170.2 92.924989) (width 0.25) (layer F.Cu) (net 19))
 (segment (start 171.17695 93.499998) (end 170.775009 93.499998) (width 0.25) (layer F.Cu) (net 19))
 (segment (start 170.2 92.14) (end 170.18 92.12) (width 0.25) (layer B.Cu) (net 19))
 (segment (start 170.2 92.924989) (end 170.2 92.14) (width 0.25) (layer B.Cu) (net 19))
 (segment (start 152.63 91.44) (end 149.925 91.44) (width 0.25) (layer F.Cu) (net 18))
 (segment (start 153.9 90.17) (end 152.63 91.44) (width 0.25) (layer F.Cu) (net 18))
 (segment (start 154.875 90.17) (end 153.9 90.17) (width 0.25) (layer F.Cu) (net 18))
 (segment (start 149.86 91.505) (end 149.925 91.44) (width 0.25) (layer F.Cu) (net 18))
 (segment (start 149.86 96.52) (end 149.86 91.505) (width 0.25) (layer F.Cu) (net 18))
 (segment (start 155.251768 90.17) (end 154.875 90.17) (width 0.25) (layer F.Cu) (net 18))
 (segment (start 167.926997 94.499999) (end 171.17695 94.499999) (width 0.25) (layer F.Cu) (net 18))
 (segment (start 167.401997 93.974999) (end 167.926997 94.499999) (width 0.25) (layer F.Cu) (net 18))
 (segment (start 166.974999 93.974999) (end 167.401997 93.974999) (width 0.25) (layer F.Cu) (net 18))
 (segment (start 165.195021 92.195021) (end 166.974999 93.974999) (width 0.25) (layer F.Cu) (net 18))
 (segment (start 159.180379 92.195021) (end 165.195021 92.195021) (width 0.25) (layer F.Cu) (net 18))
 (segment (start 157.155358 90.17) (end 159.180379 92.195021) (width 0.25) (layer F.Cu) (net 18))
 (segment (start 154.875 90.17) (end 157.155358 90.17) (width 0.25) (layer F.Cu) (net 18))
 (segment (start 152.17 88.9) (end 154.875 88.9) (width 0.25) (layer F.Cu) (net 17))
 (segment (start 150.9 90.17) (end 152.17 88.9) (width 0.25) (layer F.Cu) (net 17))
 (segment (start 149.925 90.17) (end 150.9 90.17) (width 0.25) (layer F.Cu) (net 17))
 (segment (start 148.95 90.17) (end 149.925 90.17) (width 0.25) (layer F.Cu) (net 17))
 (segment (start 148.62499 90.49501) (end 148.95 90.17) (width 0.25) (layer F.Cu) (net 17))
 (segment (start 148.62499 96.949992) (end 148.62499 90.49501) (width 0.25) (layer F.Cu) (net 17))
 (segment (start 149.319999 97.645001) (end 148.62499 96.949992) (width 0.25) (layer F.Cu) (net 17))
 (segment (start 153.814999 97.645001) (end 149.319999 97.645001) (width 0.25) (layer F.Cu) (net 17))
 (segment (start 154.94 96.52) (end 153.814999 97.645001) (width 0.25) (layer F.Cu) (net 17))
 (segment (start 155.460002 95.999998) (end 154.94 96.52) (width 0.25) (layer F.Cu) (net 17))
 (segment (start 171.17695 95.999998) (end 155.460002 95.999998) (width 0.25) (layer F.Cu) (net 17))
 (segment (start 150.665685 88.9) (end 149.925 88.9) (width 0.25) (layer F.Cu) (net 15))
 (via (at 173.9 98.4) (size 0.8) (drill 0.4) (layers F.Cu B.Cu) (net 15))
 (segment (start 173.449099 97.949099) (end 173.9 98.4) (width 0.25) (layer F.Cu) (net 15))
 (segment (start 173.449099 96.575001) (end 173.449099 97.949099) (width 0.25) (layer F.Cu) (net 15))
 (segment (start 173.5241 96.5) (end 173.449099 96.575001) (width 0.25) (layer F.Cu) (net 15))
 (segment (start 174.26305 96.5) (end 173.5241 96.5) (width 0.25) (layer F.Cu) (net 15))
 (segment (start 173.9 98.4) (end 149.2 98.4) (width 0.25) (layer B.Cu) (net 15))
 (segment (start 149.2 98.4) (end 146.9 96.1) (width 0.25) (layer B.Cu) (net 15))
 (via (at 146.9 88.9) (size 0.8) (drill 0.4) (layers F.Cu B.Cu) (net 15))
 (segment (start 146.9 96.1) (end 146.9 88.9) (width 0.25) (layer B.Cu) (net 15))
 (segment (start 146.9 88.9) (end 149.925 88.9) (width 0.25) (layer F.Cu) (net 15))
 (segment (start 155.888178 87.63) (end 154.875 87.63) (width 0.25) (layer F.Cu) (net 14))
 (segment (start 172.74859 91.295001) (end 159.553179 91.295001) (width 0.25) (layer F.Cu) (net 14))
 (segment (start 173.453608 92.000019) (end 172.74859 91.295001) (width 0.25) (layer F.Cu) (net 14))
 (segment (start 173.989421 92.00002) (end 173.453608 92.000019) (width 0.25) (layer F.Cu) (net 14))
 (segment (start 175.077001 93.0876) (end 173.989421 92.00002) (width 0.25) (layer F.Cu) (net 14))
 (segment (start 175.077001 94.912403) (end 175.077001 93.0876) (width 0.25) (layer F.Cu) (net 14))
 (segment (start 159.553179 91.295001) (end 155.888178 87.63) (width 0.25) (layer F.Cu) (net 14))
 (segment (start 174.989404 95) (end 175.077001 94.912403) (width 0.25) (layer F.Cu) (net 14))
 (segment (start 174.26305 95) (end 174.989404 95) (width 0.25) (layer F.Cu) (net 14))
 (segment (start 172.903304 94) (end 171.378303 92.474999) (width 0.25) (layer F.Cu) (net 13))
 (segment (start 174.26305 94) (end 172.903304 94) (width 0.25) (layer F.Cu) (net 13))
 (via (at 167.126998 92.674694) (size 0.8) (drill 0.4) (layers F.Cu B.Cu) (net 13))
 (segment (start 167.601704 92.199988) (end 167.126998 92.674694) (width 0.25) (layer F.Cu) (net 13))
 (segment (start 171.103292 92.199988) (end 167.601704 92.199988) (width 0.25) (layer F.Cu) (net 13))
 (segment (start 171.378303 92.474999) (end 171.103292 92.199988) (width 0.25) (layer F.Cu) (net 13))
 (segment (start 167.64 92.161692) (end 167.64 77.47) (width 0.25) (layer B.Cu) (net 13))
 (segment (start 167.126998 92.674694) (end 167.64 92.161692) (width 0.25) (layer B.Cu) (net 13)))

